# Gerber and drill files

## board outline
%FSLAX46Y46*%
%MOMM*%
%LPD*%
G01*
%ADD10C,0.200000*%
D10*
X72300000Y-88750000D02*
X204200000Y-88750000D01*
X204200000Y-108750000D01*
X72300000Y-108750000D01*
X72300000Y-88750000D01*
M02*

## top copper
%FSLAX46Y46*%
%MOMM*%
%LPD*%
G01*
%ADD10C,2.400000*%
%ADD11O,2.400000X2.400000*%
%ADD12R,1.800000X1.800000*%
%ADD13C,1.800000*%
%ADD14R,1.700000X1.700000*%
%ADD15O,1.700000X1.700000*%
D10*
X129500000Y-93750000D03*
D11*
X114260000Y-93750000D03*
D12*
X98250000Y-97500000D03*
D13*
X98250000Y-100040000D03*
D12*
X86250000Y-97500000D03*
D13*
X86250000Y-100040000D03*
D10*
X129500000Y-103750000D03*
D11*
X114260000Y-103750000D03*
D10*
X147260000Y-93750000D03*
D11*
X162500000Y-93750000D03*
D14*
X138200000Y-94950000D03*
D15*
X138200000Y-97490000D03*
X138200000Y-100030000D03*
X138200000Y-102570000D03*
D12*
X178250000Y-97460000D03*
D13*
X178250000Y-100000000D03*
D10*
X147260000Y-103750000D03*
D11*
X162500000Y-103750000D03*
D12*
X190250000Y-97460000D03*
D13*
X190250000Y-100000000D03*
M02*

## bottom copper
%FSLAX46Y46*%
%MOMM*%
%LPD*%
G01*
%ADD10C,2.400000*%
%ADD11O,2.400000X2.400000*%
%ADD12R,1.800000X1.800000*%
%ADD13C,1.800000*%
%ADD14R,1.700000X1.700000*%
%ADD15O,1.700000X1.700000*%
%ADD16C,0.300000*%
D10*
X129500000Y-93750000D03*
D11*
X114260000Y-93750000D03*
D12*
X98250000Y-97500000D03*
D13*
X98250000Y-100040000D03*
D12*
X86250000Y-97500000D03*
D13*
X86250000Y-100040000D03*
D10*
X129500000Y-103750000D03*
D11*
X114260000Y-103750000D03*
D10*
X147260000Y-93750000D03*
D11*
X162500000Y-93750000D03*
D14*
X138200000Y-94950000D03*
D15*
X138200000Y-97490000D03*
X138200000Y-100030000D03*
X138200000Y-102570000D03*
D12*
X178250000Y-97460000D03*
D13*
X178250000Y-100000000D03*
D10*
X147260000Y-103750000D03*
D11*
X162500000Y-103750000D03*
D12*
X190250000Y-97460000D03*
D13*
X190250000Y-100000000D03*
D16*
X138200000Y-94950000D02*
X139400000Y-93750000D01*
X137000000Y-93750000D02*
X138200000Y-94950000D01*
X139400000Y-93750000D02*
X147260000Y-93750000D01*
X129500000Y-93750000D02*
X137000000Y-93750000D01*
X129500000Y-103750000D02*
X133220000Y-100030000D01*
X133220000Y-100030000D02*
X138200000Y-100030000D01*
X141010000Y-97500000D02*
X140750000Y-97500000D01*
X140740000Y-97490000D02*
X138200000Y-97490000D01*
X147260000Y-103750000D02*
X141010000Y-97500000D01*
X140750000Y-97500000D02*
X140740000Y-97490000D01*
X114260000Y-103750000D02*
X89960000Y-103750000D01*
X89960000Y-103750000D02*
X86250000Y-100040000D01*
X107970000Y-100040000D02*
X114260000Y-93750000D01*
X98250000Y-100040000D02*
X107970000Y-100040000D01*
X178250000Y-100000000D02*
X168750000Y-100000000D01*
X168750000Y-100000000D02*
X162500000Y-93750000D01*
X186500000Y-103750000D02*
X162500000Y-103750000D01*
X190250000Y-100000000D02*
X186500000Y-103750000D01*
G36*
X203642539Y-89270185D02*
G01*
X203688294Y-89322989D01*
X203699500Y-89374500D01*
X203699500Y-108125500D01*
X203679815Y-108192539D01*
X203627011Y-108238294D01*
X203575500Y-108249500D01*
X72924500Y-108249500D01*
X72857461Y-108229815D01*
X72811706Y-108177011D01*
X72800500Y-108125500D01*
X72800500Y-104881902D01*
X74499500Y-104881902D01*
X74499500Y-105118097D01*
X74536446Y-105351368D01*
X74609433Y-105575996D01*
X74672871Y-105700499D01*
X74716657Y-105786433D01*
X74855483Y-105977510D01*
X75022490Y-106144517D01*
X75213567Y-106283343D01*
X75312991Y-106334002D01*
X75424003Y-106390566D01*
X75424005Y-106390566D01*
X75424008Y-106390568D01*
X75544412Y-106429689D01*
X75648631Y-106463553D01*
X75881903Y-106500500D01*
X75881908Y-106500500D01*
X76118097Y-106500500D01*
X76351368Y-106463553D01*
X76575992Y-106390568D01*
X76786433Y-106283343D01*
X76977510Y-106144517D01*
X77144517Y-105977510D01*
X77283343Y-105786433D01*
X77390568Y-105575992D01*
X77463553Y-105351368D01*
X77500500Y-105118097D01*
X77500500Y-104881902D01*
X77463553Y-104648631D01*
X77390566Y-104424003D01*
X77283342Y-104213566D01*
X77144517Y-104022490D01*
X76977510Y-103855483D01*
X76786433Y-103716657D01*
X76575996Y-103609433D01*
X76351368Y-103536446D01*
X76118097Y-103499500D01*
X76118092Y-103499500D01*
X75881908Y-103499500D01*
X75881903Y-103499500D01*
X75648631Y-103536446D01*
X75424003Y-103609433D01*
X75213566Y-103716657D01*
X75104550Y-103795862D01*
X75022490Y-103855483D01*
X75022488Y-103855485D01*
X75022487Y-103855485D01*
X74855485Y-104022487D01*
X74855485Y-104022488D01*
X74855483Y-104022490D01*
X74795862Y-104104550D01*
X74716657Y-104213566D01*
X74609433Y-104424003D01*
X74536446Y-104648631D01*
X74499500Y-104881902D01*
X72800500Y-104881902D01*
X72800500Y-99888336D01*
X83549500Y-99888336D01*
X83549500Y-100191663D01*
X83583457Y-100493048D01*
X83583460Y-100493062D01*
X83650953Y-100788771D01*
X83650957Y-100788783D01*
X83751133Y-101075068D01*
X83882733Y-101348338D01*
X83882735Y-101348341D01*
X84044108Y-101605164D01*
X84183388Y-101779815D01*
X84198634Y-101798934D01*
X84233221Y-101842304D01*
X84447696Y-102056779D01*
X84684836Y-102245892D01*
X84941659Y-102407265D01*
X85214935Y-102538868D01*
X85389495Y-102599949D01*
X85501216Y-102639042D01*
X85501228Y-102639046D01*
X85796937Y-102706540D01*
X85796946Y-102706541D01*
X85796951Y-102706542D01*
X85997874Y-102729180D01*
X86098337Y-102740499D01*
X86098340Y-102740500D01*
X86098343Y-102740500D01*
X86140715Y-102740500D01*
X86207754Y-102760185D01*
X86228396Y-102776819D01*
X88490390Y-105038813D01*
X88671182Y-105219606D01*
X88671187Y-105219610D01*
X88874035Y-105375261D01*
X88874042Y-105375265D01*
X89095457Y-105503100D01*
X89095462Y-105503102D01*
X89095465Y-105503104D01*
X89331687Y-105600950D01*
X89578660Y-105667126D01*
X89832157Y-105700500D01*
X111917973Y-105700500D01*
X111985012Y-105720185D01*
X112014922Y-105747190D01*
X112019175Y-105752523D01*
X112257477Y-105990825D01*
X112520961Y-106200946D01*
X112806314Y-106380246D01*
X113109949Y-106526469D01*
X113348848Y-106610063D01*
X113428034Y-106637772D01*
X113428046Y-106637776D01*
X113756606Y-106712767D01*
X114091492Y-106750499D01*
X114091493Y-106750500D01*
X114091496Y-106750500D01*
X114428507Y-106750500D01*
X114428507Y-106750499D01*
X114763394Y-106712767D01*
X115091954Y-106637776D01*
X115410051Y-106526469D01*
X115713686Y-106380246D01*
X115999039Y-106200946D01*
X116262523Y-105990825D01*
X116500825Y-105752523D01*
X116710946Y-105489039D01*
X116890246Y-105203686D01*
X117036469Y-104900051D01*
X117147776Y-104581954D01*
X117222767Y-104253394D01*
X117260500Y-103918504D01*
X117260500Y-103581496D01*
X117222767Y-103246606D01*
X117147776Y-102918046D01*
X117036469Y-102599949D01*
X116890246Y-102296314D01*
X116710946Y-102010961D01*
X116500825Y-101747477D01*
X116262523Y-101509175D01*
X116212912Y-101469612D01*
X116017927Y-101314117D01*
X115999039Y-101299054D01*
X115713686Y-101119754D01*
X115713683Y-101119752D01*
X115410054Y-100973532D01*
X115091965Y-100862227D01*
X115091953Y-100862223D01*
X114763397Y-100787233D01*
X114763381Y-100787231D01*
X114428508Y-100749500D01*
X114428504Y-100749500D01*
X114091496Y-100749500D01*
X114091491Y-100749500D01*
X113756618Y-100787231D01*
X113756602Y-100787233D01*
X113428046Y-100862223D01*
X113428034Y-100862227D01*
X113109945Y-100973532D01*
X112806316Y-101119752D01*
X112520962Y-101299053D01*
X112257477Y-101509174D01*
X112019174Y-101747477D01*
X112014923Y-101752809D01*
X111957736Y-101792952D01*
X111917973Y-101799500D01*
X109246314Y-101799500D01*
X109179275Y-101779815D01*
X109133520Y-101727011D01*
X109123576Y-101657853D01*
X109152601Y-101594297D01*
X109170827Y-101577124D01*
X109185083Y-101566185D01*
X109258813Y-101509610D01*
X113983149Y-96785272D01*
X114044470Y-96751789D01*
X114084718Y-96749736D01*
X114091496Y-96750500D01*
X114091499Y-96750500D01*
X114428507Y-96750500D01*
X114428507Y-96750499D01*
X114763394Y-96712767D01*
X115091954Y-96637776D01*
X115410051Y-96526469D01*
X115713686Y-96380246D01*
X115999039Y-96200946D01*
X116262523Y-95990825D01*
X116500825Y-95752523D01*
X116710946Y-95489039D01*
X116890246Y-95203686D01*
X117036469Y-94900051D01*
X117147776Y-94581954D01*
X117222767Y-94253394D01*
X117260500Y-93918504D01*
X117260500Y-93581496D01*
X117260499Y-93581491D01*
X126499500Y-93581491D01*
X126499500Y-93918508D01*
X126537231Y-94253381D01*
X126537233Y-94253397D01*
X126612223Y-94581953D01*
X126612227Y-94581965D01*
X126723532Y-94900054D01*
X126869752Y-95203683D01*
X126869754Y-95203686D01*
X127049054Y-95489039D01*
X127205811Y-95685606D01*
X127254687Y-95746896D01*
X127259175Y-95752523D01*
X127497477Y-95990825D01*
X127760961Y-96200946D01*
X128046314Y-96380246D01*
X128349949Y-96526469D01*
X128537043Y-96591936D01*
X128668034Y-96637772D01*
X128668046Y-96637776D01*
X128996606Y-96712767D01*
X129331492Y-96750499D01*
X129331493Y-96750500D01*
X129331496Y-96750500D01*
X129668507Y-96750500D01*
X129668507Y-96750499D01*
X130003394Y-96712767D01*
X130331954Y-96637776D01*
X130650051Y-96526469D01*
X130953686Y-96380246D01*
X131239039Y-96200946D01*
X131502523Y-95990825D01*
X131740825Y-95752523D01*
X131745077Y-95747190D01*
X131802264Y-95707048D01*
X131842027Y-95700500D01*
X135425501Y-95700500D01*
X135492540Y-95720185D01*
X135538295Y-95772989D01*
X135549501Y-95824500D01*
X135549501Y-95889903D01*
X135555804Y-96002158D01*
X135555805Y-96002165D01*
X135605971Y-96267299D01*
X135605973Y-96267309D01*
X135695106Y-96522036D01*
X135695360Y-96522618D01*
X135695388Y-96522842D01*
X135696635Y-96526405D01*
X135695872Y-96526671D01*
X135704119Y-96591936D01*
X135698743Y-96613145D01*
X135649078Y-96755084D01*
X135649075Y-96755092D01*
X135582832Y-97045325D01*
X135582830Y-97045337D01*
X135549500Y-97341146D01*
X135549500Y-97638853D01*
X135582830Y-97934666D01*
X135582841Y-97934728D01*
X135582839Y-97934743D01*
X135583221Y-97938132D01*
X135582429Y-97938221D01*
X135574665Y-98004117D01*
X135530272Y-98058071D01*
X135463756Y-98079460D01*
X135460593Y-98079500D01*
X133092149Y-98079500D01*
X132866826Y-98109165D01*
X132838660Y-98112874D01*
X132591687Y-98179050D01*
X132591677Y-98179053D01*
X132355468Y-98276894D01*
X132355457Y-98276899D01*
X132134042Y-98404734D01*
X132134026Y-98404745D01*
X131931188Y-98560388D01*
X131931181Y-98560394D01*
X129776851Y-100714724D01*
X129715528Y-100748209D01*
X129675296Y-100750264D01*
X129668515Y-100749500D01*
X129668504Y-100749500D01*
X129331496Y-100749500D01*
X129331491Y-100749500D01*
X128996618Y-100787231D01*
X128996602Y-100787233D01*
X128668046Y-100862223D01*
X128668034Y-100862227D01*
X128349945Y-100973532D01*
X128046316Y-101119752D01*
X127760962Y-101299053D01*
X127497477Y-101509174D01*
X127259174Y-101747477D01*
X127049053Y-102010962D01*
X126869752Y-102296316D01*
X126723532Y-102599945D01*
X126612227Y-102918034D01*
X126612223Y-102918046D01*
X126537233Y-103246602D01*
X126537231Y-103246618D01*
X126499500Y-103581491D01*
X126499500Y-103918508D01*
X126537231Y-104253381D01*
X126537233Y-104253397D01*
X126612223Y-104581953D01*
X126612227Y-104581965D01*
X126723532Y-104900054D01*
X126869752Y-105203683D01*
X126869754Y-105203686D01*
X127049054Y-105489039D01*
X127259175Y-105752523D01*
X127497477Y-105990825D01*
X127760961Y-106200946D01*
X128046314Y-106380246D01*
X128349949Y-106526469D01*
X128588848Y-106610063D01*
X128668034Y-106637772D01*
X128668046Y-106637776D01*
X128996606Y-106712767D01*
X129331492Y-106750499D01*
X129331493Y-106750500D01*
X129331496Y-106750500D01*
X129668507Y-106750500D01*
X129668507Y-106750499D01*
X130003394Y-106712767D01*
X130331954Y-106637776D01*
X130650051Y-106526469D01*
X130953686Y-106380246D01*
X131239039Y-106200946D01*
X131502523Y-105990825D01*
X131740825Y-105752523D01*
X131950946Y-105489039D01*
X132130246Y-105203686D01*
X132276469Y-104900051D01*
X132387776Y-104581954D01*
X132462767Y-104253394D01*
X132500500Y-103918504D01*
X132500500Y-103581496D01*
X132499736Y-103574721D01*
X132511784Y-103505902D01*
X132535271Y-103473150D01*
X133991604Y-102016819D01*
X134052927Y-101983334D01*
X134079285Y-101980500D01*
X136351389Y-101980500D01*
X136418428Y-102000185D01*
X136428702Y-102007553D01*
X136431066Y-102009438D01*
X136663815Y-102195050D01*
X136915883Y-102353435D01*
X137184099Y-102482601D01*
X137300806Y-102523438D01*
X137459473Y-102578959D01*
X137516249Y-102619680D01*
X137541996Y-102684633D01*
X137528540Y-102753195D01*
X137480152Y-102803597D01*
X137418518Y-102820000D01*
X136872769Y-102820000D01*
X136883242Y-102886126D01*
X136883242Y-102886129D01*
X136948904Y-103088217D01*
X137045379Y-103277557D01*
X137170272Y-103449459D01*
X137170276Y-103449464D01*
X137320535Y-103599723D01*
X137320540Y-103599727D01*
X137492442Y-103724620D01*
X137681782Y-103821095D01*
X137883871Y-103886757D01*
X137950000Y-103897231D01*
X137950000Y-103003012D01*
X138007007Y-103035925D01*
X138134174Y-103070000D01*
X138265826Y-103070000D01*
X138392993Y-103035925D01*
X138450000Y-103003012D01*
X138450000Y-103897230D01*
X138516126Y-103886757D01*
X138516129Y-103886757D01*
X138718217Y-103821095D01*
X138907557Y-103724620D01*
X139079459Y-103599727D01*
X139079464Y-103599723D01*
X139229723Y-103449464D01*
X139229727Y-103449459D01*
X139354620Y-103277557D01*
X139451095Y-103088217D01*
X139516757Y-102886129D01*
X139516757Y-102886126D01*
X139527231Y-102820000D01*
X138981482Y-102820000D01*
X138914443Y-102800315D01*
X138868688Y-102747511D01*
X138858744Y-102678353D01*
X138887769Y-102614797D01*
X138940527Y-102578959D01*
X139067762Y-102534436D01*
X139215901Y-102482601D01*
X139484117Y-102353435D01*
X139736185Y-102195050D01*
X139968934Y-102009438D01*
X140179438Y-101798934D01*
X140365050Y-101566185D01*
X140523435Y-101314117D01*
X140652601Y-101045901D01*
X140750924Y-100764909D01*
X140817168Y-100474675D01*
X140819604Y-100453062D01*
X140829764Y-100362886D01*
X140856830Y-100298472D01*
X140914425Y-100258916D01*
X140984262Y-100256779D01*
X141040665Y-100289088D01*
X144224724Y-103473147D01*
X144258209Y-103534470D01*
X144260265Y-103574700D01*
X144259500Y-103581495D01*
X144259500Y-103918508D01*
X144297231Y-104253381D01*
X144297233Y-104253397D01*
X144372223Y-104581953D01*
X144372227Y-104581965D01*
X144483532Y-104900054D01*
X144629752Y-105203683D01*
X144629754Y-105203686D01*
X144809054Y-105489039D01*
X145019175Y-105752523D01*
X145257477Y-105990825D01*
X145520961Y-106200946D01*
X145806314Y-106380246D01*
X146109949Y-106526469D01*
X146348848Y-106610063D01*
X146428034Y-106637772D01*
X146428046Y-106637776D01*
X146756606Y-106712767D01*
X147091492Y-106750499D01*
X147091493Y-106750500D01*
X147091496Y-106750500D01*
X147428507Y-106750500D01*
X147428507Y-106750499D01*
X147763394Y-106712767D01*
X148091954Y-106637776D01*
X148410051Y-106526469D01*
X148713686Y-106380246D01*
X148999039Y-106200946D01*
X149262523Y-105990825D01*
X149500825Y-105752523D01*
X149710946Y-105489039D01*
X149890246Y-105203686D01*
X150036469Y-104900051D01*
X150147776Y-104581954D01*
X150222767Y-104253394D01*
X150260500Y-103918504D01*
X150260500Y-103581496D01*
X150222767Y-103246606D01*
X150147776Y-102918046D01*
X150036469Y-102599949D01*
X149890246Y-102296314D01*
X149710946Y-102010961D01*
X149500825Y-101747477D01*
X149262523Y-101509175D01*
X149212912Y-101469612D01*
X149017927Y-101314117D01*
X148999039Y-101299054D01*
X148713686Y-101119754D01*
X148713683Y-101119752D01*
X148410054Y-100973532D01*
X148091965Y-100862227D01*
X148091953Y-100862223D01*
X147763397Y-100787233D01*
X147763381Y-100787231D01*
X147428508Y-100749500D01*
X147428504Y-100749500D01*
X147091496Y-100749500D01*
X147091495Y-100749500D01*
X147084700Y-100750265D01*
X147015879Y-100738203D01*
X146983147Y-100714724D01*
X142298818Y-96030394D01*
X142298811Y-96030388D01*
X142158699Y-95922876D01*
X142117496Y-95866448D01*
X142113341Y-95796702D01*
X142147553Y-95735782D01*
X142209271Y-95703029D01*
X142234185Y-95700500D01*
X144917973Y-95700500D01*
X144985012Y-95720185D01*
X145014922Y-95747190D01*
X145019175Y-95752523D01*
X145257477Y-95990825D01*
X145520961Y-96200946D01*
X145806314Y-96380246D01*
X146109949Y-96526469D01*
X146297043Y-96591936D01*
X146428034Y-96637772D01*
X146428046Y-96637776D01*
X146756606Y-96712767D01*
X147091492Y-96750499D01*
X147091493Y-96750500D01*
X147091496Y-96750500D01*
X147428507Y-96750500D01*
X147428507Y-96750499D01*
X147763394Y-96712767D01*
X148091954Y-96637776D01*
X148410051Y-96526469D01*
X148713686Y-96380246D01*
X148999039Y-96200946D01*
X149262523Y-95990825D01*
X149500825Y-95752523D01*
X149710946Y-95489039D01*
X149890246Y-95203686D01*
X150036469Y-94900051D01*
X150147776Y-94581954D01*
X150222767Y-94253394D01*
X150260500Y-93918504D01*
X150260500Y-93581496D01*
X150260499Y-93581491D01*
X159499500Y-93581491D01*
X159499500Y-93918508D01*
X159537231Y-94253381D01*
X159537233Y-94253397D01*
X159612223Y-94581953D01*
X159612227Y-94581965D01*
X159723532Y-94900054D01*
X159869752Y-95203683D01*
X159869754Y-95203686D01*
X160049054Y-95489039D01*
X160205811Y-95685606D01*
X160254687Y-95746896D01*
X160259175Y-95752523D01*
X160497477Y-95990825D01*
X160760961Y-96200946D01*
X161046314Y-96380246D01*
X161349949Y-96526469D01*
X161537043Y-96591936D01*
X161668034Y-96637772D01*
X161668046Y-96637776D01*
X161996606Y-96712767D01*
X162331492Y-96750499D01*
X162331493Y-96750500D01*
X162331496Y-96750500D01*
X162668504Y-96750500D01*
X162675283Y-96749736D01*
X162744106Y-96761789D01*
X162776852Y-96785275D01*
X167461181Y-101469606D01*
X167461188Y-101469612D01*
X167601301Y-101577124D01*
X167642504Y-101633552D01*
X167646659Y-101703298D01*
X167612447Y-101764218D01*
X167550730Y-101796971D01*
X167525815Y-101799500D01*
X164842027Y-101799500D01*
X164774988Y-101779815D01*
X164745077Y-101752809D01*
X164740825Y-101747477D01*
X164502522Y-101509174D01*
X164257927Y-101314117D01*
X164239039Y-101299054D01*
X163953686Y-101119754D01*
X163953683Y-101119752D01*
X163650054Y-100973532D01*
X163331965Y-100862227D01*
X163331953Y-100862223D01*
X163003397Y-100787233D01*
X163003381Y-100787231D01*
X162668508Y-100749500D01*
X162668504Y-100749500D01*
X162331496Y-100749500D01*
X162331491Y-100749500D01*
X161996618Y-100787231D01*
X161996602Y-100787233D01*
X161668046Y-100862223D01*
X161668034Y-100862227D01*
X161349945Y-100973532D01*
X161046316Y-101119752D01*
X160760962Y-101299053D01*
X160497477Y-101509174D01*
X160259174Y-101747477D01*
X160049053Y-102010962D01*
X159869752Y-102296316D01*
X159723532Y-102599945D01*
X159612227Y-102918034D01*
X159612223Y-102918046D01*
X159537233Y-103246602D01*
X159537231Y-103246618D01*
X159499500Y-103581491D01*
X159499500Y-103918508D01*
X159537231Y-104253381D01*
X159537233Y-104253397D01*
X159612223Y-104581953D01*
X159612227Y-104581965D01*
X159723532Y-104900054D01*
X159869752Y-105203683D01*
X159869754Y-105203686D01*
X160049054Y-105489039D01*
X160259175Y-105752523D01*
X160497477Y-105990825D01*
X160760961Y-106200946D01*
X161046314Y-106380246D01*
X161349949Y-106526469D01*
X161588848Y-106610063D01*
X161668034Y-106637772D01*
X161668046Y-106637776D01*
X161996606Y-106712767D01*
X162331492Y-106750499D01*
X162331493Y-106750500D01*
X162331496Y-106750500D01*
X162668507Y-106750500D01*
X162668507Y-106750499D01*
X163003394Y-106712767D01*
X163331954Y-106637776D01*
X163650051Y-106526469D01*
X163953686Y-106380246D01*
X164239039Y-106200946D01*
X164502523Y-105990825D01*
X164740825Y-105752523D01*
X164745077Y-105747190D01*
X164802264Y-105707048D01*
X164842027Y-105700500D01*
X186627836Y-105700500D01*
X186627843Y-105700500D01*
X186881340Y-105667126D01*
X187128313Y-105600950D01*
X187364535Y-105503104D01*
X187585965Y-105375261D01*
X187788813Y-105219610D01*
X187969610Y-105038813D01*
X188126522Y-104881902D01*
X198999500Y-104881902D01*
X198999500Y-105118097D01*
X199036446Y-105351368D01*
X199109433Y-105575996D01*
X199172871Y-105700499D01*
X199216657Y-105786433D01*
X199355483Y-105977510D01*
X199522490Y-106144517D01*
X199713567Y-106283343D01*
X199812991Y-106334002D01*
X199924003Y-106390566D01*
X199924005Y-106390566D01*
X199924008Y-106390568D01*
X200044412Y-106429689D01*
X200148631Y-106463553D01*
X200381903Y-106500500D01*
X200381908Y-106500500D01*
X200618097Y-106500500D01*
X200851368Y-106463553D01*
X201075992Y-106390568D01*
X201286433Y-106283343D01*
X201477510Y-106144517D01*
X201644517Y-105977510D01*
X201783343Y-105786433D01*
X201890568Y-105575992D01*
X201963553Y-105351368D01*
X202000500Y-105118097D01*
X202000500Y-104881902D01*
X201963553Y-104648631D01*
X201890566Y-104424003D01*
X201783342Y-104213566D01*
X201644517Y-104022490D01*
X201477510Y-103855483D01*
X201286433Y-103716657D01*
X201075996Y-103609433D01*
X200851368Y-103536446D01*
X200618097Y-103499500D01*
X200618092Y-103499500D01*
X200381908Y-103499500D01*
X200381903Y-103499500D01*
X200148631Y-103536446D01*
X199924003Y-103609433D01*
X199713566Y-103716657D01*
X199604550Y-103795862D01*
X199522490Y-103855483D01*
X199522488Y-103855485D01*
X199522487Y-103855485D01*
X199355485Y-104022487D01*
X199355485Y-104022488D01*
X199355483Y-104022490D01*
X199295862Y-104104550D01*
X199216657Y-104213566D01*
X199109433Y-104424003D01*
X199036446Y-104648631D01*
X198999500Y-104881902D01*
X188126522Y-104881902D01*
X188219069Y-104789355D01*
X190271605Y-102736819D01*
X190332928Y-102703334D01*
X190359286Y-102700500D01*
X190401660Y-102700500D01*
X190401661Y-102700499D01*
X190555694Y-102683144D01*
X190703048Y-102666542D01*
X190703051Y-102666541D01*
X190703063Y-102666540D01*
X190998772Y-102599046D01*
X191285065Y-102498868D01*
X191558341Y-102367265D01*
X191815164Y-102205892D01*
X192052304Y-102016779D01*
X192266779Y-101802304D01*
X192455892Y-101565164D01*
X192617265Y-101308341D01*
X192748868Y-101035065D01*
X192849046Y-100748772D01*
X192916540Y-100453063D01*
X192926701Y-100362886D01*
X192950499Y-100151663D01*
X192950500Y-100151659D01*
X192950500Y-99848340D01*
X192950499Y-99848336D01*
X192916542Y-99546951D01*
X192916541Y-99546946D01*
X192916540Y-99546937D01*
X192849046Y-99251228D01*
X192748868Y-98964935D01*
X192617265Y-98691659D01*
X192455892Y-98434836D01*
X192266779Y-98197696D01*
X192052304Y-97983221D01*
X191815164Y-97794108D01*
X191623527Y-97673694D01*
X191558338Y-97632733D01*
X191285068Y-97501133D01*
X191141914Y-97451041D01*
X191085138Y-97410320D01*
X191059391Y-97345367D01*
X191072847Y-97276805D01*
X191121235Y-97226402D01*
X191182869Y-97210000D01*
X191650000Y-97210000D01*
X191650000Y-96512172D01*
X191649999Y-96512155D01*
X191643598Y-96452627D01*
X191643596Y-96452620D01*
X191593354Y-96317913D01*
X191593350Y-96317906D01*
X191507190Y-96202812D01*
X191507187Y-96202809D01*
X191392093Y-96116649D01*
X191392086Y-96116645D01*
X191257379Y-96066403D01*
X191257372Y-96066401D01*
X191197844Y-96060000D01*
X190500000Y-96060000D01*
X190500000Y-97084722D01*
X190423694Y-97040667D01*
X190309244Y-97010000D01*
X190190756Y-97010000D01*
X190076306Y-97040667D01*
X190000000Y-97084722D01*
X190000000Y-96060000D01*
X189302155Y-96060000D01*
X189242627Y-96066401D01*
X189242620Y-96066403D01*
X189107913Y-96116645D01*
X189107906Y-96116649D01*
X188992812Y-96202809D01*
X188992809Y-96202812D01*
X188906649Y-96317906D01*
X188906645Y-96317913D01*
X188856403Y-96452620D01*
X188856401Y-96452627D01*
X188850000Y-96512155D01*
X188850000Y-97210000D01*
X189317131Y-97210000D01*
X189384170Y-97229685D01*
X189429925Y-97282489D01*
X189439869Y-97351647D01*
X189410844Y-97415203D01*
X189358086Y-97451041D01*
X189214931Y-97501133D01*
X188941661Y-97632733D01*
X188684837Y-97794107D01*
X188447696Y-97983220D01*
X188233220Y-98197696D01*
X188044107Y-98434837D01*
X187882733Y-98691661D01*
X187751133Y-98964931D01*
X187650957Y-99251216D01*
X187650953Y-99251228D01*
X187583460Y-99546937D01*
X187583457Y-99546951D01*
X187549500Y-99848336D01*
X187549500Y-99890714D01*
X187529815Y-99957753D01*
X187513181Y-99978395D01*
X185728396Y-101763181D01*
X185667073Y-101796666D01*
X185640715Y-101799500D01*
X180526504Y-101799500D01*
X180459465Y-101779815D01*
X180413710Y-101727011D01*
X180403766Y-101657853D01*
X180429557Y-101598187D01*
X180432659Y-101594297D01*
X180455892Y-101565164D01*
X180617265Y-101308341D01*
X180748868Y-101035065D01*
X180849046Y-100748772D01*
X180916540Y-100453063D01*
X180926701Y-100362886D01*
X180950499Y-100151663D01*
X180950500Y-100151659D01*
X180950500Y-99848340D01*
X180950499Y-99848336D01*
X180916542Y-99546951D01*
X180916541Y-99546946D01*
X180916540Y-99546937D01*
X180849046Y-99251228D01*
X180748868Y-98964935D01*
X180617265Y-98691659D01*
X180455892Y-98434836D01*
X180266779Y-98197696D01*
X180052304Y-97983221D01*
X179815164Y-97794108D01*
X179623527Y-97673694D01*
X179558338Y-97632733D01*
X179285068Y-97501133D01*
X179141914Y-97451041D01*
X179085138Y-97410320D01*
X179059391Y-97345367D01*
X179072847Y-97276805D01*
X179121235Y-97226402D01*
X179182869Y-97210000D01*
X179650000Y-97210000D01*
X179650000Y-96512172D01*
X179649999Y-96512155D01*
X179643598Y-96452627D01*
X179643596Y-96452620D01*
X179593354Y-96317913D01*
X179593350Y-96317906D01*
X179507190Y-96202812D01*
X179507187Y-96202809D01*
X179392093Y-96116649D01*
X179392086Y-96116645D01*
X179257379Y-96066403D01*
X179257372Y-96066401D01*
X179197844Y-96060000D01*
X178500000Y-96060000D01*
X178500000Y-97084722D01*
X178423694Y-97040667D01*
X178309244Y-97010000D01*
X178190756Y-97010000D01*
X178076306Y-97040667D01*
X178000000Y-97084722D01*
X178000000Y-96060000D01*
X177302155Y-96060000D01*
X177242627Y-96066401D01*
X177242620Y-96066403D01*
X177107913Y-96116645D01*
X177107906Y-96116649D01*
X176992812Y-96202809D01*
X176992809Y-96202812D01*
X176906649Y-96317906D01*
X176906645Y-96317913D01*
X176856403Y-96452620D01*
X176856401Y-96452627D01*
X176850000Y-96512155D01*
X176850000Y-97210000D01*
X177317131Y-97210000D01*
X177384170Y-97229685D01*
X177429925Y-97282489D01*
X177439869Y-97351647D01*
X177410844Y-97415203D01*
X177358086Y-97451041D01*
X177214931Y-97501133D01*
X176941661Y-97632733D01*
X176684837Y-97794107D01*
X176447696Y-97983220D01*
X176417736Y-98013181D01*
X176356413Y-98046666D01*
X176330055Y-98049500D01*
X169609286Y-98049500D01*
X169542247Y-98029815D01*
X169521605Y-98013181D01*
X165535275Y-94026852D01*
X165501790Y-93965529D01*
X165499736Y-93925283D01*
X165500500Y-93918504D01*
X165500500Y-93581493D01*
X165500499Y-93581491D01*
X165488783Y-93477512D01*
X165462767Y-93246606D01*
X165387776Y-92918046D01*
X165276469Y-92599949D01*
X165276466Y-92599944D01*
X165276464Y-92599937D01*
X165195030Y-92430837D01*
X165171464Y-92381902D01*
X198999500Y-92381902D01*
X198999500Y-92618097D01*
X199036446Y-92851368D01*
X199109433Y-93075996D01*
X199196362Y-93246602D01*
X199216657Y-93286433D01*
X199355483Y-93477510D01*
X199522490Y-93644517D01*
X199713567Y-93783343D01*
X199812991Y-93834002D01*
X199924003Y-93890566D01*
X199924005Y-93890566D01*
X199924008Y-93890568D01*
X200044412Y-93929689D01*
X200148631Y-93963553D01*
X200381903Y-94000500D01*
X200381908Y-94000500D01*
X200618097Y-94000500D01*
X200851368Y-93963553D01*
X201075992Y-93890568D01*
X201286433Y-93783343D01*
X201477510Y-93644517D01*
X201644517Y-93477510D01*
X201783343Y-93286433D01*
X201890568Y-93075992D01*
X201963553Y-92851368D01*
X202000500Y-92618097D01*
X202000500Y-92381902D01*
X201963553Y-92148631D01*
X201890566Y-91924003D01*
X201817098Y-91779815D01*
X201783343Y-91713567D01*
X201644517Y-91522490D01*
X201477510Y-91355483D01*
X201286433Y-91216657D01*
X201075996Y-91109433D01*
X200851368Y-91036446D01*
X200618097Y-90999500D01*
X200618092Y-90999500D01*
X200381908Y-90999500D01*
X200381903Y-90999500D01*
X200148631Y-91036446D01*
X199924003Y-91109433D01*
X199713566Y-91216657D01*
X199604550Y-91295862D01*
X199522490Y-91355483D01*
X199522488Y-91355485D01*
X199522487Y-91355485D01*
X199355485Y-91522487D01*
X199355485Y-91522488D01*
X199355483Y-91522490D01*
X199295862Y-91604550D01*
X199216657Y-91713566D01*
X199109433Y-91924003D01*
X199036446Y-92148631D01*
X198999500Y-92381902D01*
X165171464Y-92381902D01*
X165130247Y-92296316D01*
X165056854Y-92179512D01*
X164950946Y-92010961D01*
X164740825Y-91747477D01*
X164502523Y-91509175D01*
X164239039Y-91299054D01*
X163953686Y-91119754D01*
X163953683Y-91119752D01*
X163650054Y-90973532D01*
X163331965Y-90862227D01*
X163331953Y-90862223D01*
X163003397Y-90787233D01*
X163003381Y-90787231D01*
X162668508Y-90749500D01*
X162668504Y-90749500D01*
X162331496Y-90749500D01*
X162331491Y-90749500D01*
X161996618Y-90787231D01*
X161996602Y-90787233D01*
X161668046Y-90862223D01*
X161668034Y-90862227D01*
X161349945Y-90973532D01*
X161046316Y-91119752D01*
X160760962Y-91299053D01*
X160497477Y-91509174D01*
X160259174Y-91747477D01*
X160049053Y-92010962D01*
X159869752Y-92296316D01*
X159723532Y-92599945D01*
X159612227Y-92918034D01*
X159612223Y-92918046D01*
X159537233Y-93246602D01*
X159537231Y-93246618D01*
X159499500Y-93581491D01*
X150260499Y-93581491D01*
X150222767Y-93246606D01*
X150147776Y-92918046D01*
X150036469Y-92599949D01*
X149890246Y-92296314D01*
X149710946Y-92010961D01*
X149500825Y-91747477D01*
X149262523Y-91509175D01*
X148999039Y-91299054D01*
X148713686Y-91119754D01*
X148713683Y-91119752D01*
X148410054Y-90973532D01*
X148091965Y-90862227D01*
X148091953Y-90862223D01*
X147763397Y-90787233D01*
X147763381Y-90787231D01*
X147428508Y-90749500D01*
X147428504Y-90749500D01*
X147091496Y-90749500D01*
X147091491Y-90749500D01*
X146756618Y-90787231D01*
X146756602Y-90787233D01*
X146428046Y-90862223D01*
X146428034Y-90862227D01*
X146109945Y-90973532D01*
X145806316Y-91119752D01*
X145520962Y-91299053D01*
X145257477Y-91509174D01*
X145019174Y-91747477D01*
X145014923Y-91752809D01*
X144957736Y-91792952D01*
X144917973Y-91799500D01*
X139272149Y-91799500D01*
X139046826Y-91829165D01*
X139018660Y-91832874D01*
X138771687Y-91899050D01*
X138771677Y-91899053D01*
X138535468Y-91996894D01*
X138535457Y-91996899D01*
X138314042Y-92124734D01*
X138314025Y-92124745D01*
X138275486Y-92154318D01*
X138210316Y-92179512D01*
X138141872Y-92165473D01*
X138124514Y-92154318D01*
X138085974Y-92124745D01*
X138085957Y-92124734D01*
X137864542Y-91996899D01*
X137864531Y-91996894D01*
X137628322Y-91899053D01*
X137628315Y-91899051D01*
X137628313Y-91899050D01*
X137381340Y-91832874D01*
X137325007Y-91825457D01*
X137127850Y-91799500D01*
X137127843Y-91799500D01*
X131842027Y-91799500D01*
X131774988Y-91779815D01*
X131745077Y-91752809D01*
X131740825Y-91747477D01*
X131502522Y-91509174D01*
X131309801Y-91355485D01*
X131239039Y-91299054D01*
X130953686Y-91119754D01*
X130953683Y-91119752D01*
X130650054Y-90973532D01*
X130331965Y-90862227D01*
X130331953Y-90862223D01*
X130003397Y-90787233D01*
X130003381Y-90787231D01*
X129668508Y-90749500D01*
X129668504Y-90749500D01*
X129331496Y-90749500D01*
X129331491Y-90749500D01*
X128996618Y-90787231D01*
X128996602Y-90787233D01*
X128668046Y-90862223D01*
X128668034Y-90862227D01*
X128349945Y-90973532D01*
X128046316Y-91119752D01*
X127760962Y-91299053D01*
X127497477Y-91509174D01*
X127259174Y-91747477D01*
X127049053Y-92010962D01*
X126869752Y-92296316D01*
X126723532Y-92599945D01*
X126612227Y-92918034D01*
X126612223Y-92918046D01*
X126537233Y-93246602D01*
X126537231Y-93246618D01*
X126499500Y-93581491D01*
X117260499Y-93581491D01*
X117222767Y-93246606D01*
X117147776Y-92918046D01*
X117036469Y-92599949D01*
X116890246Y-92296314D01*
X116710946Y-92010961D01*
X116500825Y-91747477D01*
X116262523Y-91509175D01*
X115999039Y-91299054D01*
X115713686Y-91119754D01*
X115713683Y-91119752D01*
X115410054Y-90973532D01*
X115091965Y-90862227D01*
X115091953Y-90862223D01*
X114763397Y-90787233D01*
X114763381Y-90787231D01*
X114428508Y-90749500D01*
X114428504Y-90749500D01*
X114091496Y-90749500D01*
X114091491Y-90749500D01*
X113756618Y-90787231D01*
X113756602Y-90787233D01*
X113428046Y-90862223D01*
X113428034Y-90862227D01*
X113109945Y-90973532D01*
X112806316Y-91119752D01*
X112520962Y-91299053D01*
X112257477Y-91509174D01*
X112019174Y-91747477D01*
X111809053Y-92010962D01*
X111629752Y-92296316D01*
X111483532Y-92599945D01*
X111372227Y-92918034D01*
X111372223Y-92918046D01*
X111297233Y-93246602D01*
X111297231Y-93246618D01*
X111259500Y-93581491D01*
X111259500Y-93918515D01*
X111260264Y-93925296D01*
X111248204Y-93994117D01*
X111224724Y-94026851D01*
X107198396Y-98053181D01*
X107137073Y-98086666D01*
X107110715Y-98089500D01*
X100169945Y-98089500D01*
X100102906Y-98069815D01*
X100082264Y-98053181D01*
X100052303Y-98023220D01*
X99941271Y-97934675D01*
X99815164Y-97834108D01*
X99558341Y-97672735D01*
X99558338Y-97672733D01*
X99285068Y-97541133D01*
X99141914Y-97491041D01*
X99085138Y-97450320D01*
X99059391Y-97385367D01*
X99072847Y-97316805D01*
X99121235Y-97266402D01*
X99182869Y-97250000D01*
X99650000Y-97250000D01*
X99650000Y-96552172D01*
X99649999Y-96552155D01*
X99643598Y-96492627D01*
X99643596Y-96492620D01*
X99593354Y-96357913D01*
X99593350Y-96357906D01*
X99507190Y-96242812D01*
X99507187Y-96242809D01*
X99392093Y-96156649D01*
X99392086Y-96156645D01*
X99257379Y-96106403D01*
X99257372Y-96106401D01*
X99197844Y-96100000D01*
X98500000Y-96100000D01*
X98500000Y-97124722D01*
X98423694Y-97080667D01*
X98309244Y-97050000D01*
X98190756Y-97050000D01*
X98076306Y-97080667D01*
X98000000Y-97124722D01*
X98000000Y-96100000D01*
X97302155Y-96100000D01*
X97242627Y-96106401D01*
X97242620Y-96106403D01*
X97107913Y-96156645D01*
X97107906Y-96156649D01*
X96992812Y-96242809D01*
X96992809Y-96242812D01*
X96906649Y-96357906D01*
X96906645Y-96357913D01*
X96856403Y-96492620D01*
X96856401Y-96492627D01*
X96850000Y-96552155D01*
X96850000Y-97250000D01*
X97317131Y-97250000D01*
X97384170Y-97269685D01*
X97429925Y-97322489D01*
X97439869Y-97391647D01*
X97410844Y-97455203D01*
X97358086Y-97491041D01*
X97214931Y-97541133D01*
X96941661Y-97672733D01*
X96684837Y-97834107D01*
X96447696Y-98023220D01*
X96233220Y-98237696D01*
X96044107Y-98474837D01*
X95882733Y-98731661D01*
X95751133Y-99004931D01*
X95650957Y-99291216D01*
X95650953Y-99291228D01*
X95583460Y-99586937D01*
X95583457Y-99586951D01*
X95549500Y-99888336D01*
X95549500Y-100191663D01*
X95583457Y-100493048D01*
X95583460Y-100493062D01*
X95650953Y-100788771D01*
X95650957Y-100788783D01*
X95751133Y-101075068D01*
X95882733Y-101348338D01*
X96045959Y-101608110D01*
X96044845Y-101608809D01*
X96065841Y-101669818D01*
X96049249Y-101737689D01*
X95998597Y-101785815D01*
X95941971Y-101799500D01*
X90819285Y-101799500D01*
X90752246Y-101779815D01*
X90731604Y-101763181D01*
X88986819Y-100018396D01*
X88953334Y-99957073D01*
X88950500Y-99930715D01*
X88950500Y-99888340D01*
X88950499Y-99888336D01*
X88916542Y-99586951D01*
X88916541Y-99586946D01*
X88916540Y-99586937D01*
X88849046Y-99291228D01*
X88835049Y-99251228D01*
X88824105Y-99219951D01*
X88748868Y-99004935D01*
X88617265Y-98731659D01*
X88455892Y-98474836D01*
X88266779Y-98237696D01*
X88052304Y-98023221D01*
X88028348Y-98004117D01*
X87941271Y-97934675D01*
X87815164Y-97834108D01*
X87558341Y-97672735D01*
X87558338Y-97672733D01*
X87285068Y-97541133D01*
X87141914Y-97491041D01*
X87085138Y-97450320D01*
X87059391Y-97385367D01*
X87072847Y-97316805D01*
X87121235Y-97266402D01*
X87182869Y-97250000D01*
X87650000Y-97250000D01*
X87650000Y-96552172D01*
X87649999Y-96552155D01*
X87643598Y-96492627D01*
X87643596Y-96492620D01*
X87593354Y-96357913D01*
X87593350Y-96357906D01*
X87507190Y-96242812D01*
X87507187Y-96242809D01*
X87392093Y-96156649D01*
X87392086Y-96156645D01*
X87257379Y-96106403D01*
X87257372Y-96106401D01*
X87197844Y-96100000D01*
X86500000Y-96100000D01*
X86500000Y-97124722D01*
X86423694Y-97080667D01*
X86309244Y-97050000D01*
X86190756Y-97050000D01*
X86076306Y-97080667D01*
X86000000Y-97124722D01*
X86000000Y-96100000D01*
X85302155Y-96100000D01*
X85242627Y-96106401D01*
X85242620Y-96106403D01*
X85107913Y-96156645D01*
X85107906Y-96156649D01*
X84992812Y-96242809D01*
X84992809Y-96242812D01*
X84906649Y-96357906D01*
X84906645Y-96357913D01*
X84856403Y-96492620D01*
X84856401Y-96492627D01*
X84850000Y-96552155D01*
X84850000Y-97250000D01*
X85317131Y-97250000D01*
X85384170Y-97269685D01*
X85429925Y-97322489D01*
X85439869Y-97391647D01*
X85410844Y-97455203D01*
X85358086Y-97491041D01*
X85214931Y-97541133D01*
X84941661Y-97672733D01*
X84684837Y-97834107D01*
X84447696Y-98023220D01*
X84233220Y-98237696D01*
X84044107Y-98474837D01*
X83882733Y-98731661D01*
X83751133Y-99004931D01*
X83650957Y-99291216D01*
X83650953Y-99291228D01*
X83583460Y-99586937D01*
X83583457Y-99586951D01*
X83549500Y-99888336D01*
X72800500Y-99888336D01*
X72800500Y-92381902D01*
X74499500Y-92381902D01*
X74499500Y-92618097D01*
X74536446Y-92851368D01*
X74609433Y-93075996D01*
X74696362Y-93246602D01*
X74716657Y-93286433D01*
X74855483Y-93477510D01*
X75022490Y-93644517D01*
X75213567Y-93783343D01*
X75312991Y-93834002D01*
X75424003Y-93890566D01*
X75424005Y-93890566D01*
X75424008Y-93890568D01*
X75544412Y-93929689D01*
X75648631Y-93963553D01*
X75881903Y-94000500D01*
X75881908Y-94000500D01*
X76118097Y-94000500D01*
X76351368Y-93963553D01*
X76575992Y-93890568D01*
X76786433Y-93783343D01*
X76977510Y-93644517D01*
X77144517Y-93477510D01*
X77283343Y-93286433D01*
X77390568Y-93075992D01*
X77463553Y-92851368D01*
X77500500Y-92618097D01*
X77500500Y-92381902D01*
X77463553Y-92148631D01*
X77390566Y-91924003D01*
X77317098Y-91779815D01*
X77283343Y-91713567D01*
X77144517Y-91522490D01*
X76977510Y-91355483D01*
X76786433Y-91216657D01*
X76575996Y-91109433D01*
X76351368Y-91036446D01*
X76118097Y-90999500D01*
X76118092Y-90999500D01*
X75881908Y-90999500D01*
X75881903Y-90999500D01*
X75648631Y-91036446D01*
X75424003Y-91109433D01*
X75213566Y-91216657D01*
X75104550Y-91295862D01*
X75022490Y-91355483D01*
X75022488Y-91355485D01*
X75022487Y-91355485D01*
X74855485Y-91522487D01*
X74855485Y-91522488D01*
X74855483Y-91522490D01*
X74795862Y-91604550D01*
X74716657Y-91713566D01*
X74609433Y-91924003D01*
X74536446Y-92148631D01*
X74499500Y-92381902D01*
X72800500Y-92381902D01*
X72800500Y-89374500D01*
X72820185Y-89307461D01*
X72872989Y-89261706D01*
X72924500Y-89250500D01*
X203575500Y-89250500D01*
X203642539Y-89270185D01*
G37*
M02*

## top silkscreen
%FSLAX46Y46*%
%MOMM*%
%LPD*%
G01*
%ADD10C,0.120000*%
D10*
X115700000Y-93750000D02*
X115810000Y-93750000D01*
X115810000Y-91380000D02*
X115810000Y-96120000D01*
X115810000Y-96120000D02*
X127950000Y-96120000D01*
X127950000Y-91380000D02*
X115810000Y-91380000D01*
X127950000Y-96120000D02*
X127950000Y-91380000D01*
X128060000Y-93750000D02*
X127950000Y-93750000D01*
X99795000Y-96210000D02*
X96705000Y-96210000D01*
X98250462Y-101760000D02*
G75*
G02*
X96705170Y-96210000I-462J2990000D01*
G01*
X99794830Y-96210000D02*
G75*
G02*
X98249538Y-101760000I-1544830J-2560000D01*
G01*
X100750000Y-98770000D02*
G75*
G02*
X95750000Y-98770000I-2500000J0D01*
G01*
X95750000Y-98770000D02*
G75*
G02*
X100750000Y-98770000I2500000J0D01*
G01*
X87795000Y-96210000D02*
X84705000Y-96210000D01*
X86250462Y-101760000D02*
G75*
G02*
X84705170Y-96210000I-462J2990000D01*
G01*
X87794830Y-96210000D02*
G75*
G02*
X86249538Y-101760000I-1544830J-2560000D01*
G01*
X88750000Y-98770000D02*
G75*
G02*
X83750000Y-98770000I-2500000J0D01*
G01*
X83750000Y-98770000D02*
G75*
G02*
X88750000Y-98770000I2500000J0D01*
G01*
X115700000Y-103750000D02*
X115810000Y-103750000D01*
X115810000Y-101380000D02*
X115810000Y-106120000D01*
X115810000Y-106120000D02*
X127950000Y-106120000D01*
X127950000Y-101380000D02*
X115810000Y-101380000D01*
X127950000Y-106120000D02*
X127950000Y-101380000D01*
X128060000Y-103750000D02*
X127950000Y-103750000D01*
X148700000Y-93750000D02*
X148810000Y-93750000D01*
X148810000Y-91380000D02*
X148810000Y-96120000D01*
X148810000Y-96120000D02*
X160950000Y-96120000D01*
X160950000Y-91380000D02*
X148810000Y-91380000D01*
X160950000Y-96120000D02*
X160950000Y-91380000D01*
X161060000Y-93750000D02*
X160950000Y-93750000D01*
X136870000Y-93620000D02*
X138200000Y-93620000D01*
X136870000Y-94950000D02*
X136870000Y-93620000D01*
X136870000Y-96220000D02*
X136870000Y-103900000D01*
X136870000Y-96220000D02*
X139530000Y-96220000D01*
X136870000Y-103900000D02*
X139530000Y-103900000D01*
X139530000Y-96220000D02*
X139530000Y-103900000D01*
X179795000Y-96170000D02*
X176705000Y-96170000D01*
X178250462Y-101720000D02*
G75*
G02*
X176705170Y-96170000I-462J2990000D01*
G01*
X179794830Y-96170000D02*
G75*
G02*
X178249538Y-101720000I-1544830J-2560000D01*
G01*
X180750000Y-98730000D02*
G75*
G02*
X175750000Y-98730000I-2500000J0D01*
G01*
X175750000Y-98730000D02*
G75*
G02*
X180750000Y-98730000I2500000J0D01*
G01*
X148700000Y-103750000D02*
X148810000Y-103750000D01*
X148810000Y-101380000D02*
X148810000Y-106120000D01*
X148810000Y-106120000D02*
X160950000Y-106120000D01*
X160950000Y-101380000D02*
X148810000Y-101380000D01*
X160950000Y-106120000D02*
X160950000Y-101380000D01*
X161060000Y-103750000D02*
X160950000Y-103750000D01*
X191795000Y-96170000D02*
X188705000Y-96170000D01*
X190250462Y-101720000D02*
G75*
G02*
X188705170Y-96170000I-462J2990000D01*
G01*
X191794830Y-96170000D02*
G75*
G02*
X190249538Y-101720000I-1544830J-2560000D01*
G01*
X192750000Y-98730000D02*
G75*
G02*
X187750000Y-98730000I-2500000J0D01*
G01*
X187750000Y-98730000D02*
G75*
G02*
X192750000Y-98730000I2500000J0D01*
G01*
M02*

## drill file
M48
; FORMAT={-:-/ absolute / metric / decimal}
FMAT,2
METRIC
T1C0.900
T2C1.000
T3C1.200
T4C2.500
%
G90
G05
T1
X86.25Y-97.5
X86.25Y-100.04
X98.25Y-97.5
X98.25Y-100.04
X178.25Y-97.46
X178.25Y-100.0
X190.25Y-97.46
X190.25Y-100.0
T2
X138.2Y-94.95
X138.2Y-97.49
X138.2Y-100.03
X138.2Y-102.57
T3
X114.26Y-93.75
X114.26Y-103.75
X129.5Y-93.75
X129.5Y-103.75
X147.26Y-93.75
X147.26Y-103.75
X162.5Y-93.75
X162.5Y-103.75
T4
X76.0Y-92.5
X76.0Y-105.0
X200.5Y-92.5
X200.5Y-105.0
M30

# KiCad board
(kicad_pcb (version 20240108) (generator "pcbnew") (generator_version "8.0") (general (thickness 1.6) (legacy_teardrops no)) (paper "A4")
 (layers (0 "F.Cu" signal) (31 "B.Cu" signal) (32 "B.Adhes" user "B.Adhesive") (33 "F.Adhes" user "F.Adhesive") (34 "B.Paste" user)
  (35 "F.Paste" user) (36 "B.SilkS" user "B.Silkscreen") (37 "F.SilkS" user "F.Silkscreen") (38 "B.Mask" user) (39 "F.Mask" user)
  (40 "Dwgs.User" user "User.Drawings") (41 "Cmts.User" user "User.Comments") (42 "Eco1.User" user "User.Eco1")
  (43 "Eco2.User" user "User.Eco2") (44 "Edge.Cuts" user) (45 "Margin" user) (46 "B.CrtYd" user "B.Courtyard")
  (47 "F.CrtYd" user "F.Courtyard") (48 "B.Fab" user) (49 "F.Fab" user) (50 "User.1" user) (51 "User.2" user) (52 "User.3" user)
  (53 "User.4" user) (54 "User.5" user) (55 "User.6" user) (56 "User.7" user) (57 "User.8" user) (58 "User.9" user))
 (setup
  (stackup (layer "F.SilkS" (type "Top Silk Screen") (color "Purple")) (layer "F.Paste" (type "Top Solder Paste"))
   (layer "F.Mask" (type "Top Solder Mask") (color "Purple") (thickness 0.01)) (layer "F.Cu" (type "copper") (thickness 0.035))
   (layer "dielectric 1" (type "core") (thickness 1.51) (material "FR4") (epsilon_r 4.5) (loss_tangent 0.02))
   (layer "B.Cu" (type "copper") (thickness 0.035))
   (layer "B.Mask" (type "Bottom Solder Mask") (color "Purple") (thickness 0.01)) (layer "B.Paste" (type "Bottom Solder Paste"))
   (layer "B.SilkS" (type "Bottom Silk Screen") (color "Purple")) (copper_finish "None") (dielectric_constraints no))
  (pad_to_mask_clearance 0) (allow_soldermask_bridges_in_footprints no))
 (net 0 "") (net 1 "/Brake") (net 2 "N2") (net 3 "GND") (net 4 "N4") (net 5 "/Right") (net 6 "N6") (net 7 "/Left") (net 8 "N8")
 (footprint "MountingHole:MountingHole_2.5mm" (layer "F.Cu") (at 200.5 105)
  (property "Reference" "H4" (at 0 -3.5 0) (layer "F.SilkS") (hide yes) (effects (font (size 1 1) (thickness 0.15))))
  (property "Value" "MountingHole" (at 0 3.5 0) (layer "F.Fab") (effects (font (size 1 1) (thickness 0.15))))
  (pad "" np_thru_hole circle (at 0 0) (size 2.5 2.5) (drill 2.5) (layers "*.Cu" "*.Mask")))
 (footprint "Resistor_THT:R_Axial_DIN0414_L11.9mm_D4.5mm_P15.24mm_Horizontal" (layer "F.Cu") (at 129.5 93.75 180)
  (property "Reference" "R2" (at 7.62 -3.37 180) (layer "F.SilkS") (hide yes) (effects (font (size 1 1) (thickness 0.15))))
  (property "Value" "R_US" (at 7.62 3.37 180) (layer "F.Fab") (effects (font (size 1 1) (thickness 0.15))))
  (fp_line (start 13.8 0) (end 13.69 0) (stroke (width 0.12) (type solid)) (layer "F.SilkS"))
  (fp_line (start 13.69 2.37) (end 13.69 -2.37) (stroke (width 0.12) (type solid)) (layer "F.SilkS"))
  (fp_line (start 13.69 -2.37) (end 1.55 -2.37) (stroke (width 0.12) (type solid)) (layer "F.SilkS"))
  (fp_line (start 1.55 2.37) (end 13.69 2.37) (stroke (width 0.12) (type solid)) (layer "F.SilkS"))
  (fp_line (start 1.55 -2.37) (end 1.55 2.37) (stroke (width 0.12) (type solid)) (layer "F.SilkS"))
  (fp_line (start 1.44 0) (end 1.55 0) (stroke (width 0.12) (type solid)) (layer "F.SilkS"))
  (pad "1" thru_hole circle (at 0 0 180) (size 2.4 2.4) (drill 1.2) (layers "*.Cu" "*.Mask") (remove_unused_layers no) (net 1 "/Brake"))
  (pad "2" thru_hole oval (at 15.24 0 180) (size 2.4 2.4) (drill 1.2) (layers "*.Cu" "*.Mask") (remove_unused_layers no) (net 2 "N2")))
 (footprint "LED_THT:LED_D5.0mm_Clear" (layer "F.Cu") (at 98.25 97.5 -90)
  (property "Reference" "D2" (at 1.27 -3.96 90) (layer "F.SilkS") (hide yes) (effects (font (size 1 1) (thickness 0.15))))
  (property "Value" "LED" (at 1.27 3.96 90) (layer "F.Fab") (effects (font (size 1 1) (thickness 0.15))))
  (fp_line (start -1.29 -1.545) (end -1.29 1.545) (stroke (width 0.12) (type solid)) (layer "F.SilkS"))
  (fp_arc (start 4.26 -0.000462) (mid 2.072002 2.880433) (end -1.29 1.54483) (stroke (width 0.12) (type solid)) (layer "F.SilkS"))
  (fp_arc (start -1.29 -1.54483) (mid 2.072002 -2.880433) (end 4.26 0.000462) (stroke (width 0.12) (type solid)) (layer "F.SilkS"))
  (fp_circle (center 1.27 0) (end 3.77 0) (stroke (width 0.12) (type solid)) (fill none) (layer "F.SilkS"))
  (pad "1" thru_hole rect (at 0 0 270) (size 1.8 1.8) (drill 0.9) (layers "*.Cu" "*.Mask") (remove_unused_layers no) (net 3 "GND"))
  (pad "2" thru_hole circle (at 2.54 0 270) (size 1.8 1.8) (drill 0.9) (layers "*.Cu" "*.Mask") (remove_unused_layers no) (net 2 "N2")))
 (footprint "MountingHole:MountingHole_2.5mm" (layer "F.Cu") (at 76 92.5)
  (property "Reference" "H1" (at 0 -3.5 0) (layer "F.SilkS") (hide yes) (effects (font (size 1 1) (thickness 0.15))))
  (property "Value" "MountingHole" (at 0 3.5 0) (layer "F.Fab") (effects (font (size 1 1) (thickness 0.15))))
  (pad "" np_thru_hole circle (at 0 0) (size 2.5 2.5) (drill 2.5) (layers "*.Cu" "*.Mask")))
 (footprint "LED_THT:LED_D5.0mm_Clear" (layer "F.Cu") (at 86.25 97.5 -90)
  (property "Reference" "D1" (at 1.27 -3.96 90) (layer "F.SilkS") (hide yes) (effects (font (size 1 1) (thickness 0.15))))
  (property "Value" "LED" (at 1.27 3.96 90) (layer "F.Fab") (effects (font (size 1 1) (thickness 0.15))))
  (fp_line (start -1.29 -1.545) (end -1.29 1.545) (stroke (width 0.12) (type solid)) (layer "F.SilkS"))
  (fp_arc (start 4.26 -0.000462) (mid 2.072002 2.880433) (end -1.29 1.54483) (stroke (width 0.12) (type solid)) (layer "F.SilkS"))
  (fp_arc (start -1.29 -1.54483) (mid 2.072002 -2.880433) (end 4.26 0.000462) (stroke (width 0.12) (type solid)) (layer "F.SilkS"))
  (fp_circle (center 1.27 0) (end 3.77 0) (stroke (width 0.12) (type solid)) (fill none) (layer "F.SilkS"))
  (pad "1" thru_hole rect (at 0 0 270) (size 1.8 1.8) (drill 0.9) (layers "*.Cu" "*.Mask") (remove_unused_layers no) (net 3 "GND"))
  (pad "2" thru_hole circle (at 2.54 0 270) (size 1.8 1.8) (drill 0.9) (layers "*.Cu" "*.Mask") (remove_unused_layers no) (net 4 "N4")))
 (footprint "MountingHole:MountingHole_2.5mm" (layer "F.Cu") (at 76 105)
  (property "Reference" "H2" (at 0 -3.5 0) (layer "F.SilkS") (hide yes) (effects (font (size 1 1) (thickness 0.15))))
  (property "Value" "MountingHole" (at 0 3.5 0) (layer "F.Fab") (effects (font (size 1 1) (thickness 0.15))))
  (pad "" np_thru_hole circle (at 0 0) (size 2.5 2.5) (drill 2.5) (layers "*.Cu" "*.Mask")))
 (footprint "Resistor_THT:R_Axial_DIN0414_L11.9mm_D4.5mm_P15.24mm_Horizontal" (layer "F.Cu") (at 129.5 103.75 180)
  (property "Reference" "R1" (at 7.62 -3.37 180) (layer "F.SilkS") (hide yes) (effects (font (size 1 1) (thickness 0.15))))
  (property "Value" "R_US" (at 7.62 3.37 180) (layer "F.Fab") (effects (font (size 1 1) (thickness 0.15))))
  (fp_line (start 13.8 0) (end 13.69 0) (stroke (width 0.12) (type solid)) (layer "F.SilkS"))
  (fp_line (start 13.69 2.37) (end 13.69 -2.37) (stroke (width 0.12) (type solid)) (layer "F.SilkS"))
  (fp_line (start 13.69 -2.37) (end 1.55 -2.37) (stroke (width 0.12) (type solid)) (layer "F.SilkS"))
  (fp_line (start 1.55 2.37) (end 13.69 2.37) (stroke (width 0.12) (type solid)) (layer "F.SilkS"))
  (fp_line (start 1.55 -2.37) (end 1.55 2.37) (stroke (width 0.12) (type solid)) (layer "F.SilkS"))
  (fp_line (start 1.44 0) (end 1.55 0) (stroke (width 0.12) (type solid)) (layer "F.SilkS"))
  (pad "1" thru_hole circle (at 0 0 180) (size 2.4 2.4) (drill 1.2) (layers "*.Cu" "*.Mask") (remove_unused_layers no) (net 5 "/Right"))
  (pad "2" thru_hole oval (at 15.24 0 180) (size 2.4 2.4) (drill 1.2) (layers "*.Cu" "*.Mask") (remove_unused_layers no) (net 4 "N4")))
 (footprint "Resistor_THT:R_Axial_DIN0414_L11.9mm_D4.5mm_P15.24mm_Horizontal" (layer "F.Cu") (at 147.26 93.75)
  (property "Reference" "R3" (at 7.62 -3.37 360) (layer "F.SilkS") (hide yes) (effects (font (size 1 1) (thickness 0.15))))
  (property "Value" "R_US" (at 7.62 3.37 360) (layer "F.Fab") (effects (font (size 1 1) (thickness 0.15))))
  (fp_line (start 1.44 0) (end 1.55 0) (stroke (width 0.12) (type solid)) (layer "F.SilkS"))
  (fp_line (start 1.55 -2.37) (end 1.55 2.37) (stroke (width 0.12) (type solid)) (layer "F.SilkS"))
  (fp_line (start 1.55 2.37) (end 13.69 2.37) (stroke (width 0.12) (type solid)) (layer "F.SilkS"))
  (fp_line (start 13.69 -2.37) (end 1.55 -2.37) (stroke (width 0.12) (type solid)) (layer "F.SilkS"))
  (fp_line (start 13.69 2.37) (end 13.69 -2.37) (stroke (width 0.12) (type solid)) (layer "F.SilkS"))
  (fp_line (start 13.8 0) (end 13.69 0) (stroke (width 0.12) (type solid)) (layer "F.SilkS"))
  (pad "1" thru_hole circle (at 0 0) (size 2.4 2.4) (drill 1.2) (layers "*.Cu" "*.Mask") (remove_unused_layers no) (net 1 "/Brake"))
  (pad "2" thru_hole oval (at 15.24 0) (size 2.4 2.4) (drill 1.2) (layers "*.Cu" "*.Mask") (remove_unused_layers no) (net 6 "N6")))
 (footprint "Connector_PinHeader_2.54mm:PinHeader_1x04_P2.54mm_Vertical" (layer "F.Cu") (at 138.2 94.95)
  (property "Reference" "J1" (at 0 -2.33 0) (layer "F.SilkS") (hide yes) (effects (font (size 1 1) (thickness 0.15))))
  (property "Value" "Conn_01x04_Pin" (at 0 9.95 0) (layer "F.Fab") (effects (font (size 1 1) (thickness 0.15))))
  (fp_line (start -1.33 -1.33) (end 0 -1.33) (stroke (width 0.12) (type solid)) (layer "F.SilkS"))
  (fp_line (start -1.33 0) (end -1.33 -1.33) (stroke (width 0.12) (type solid)) (layer "F.SilkS"))
  (fp_line (start -1.33 1.27) (end -1.33 8.95) (stroke (width 0.12) (type solid)) (layer "F.SilkS"))
  (fp_line (start -1.33 1.27) (end 1.33 1.27) (stroke (width 0.12) (type solid)) (layer "F.SilkS"))
  (fp_line (start -1.33 8.95) (end 1.33 8.95) (stroke (width 0.12) (type solid)) (layer "F.SilkS"))
  (fp_line (start 1.33 1.27) (end 1.33 8.95) (stroke (width 0.12) (type solid)) (layer "F.SilkS"))
  (pad "1" thru_hole rect (at 0 0) (size 1.7 1.7) (drill 1) (layers "*.Cu" "*.Mask") (remove_unused_layers no) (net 1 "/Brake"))
  (pad "2" thru_hole oval (at 0 2.54) (size 1.7 1.7) (drill 1) (layers "*.Cu" "*.Mask") (remove_unused_layers no) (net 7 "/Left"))
  (pad "3" thru_hole oval (at 0 5.08) (size 1.7 1.7) (drill 1) (layers "*.Cu" "*.Mask") (remove_unused_layers no) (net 5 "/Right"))
  (pad "4" thru_hole oval (at 0 7.62) (size 1.7 1.7) (drill 1) (layers "*.Cu" "*.Mask") (remove_unused_layers no) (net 3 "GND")))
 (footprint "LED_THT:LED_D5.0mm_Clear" (layer "F.Cu") (at 178.25 97.46 -90)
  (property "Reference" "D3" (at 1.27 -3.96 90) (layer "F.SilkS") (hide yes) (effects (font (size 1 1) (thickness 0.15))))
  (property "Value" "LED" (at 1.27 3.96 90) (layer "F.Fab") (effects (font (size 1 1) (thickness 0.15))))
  (fp_line (start -1.29 -1.545) (end -1.29 1.545) (stroke (width 0.12) (type solid)) (layer "F.SilkS"))
  (fp_arc (start 4.26 -0.000462) (mid 2.072002 2.880433) (end -1.29 1.54483) (stroke (width 0.12) (type solid)) (layer "F.SilkS"))
  (fp_arc (start -1.29 -1.54483) (mid 2.072002 -2.880433) (end 4.26 0.000462) (stroke (width 0.12) (type solid)) (layer "F.SilkS"))
  (fp_circle (center 1.27 0) (end 3.77 0) (stroke (width 0.12) (type solid)) (fill none) (layer "F.SilkS"))
  (pad "1" thru_hole rect (at 0 0 270) (size 1.8 1.8) (drill 0.9) (layers "*.Cu" "*.Mask") (remove_unused_layers no) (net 3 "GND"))
  (pad "2" thru_hole circle (at 2.54 0 270) (size 1.8 1.8) (drill 0.9) (layers "*.Cu" "*.Mask") (remove_unused_layers no) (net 6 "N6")))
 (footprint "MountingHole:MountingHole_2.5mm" (layer "F.Cu") (at 200.5 92.5)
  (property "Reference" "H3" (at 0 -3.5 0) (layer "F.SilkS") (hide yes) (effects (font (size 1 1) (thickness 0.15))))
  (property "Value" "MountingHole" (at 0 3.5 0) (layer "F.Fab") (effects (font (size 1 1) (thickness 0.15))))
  (pad "" np_thru_hole circle (at 0 0) (size 2.5 2.5) (drill 2.5) (layers "*.Cu" "*.Mask")))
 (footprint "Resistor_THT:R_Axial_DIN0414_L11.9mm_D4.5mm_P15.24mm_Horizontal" (layer "F.Cu") (at 147.26 103.75)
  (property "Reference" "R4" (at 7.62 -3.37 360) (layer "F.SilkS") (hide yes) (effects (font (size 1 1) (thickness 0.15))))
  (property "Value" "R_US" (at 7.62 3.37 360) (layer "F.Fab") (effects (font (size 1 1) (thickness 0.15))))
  (fp_line (start 1.44 0) (end 1.55 0) (stroke (width 0.12) (type solid)) (layer "F.SilkS"))
  (fp_line (start 1.55 -2.37) (end 1.55 2.37) (stroke (width 0.12) (type solid)) (layer "F.SilkS"))
  (fp_line (start 1.55 2.37) (end 13.69 2.37) (stroke (width 0.12) (type solid)) (layer "F.SilkS"))
  (fp_line (start 13.69 -2.37) (end 1.55 -2.37) (stroke (width 0.12) (type solid)) (layer "F.SilkS"))
  (fp_line (start 13.69 2.37) (end 13.69 -2.37) (stroke (width 0.12) (type solid)) (layer "F.SilkS"))
  (fp_line (start 13.8 0) (end 13.69 0) (stroke (width 0.12) (type solid)) (layer "F.SilkS"))
  (pad "1" thru_hole circle (at 0 0) (size 2.4 2.4) (drill 1.2) (layers "*.Cu" "*.Mask") (remove_unused_layers no) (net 7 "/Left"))
  (pad "2" thru_hole oval (at 15.24 0) (size 2.4 2.4) (drill 1.2) (layers "*.Cu" "*.Mask") (remove_unused_layers no) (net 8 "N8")))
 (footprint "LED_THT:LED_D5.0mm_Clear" (layer "F.Cu") (at 190.25 97.46 -90)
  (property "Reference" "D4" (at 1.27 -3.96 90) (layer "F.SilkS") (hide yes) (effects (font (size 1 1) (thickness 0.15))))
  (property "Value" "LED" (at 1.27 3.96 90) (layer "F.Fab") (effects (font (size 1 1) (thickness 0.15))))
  (fp_line (start -1.29 -1.545) (end -1.29 1.545) (stroke (width 0.12) (type solid)) (layer "F.SilkS"))
  (fp_arc (start 4.26 -0.000462) (mid 2.072002 2.880433) (end -1.29 1.54483) (stroke (width 0.12) (type solid)) (layer "F.SilkS"))
  (fp_arc (start -1.29 -1.54483) (mid 2.072002 -2.880433) (end 4.26 0.000462) (stroke (width 0.12) (type solid)) (layer "F.SilkS"))
  (fp_circle (center 1.27 0) (end 3.77 0) (stroke (width 0.12) (type solid)) (fill none) (layer "F.SilkS"))
  (pad "1" thru_hole rect (at 0 0 270) (size 1.8 1.8) (drill 0.9) (layers "*.Cu" "*.Mask") (remove_unused_layers no) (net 3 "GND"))
  (pad "2" thru_hole circle (at 2.54 0 270) (size 1.8 1.8) (drill 0.9) (layers "*.Cu" "*.Mask") (remove_unused_layers no) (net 8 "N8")))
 (gr_rect (start 72.3 88.75) (end 204.2 108.75) (stroke (width 0.2) (type default)) (fill none) (layer "Edge.Cuts"))
 (segment (start 138.2 94.95) (end 139.4 93.75) (width 0.3) (layer "B.Cu") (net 1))
 (segment (start 137 93.75) (end 138.2 94.95) (width 0.3) (layer "B.Cu") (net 1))
 (segment (start 139.4 93.75) (end 147.26 93.75) (width 0.3) (layer "B.Cu") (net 1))
 (segment (start 129.5 93.75) (end 137 93.75) (width 0.3) (layer "B.Cu") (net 1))
 (segment (start 129.5 103.75) (end 133.22 100.03) (width 0.3) (layer "B.Cu") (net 5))
 (segment (start 133.22 100.03) (end 138.2 100.03) (width 0.3) (layer "B.Cu") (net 5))
 (segment (start 141.01 97.5) (end 140.75 97.5) (width 0.3) (layer "B.Cu") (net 7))
 (segment (start 140.74 97.49) (end 138.2 97.49) (width 0.3) (layer "B.Cu") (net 7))
 (segment (start 147.26 103.75) (end 141.01 97.5) (width 0.3) (layer "B.Cu") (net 7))
 (segment (start 140.75 97.5) (end 140.74 97.49) (width 0.3) (layer "B.Cu") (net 7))
 (segment (start 114.26 103.75) (end 89.96 103.75) (width 0.3) (layer "B.Cu") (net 4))
 (segment (start 89.96 103.75) (end 86.25 100.04) (width 0.3) (layer "B.Cu") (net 4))
 (segment (start 107.97 100.04) (end 114.26 93.75) (width 0.3) (layer "B.Cu") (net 2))
 (segment (start 98.25 100.04) (end 107.97 100.04) (width 0.3) (layer "B.Cu") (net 2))
 (segment (start 178.25 100) (end 168.75 100) (width 0.3) (layer "B.Cu") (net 6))
 (segment (start 168.75 100) (end 162.5 93.75) (width 0.3) (layer "B.Cu") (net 6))
 (segment (start 186.5 103.75) (end 162.5 103.75) (width 0.3) (layer "B.Cu") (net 8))
 (segment (start 190.25 100) (end 186.5 103.75) (width 0.3) (layer "B.Cu") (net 8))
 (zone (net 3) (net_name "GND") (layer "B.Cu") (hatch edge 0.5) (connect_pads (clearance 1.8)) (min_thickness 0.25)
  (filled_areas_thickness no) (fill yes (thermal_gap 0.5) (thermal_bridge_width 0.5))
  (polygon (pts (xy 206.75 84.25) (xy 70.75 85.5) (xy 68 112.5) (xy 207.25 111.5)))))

